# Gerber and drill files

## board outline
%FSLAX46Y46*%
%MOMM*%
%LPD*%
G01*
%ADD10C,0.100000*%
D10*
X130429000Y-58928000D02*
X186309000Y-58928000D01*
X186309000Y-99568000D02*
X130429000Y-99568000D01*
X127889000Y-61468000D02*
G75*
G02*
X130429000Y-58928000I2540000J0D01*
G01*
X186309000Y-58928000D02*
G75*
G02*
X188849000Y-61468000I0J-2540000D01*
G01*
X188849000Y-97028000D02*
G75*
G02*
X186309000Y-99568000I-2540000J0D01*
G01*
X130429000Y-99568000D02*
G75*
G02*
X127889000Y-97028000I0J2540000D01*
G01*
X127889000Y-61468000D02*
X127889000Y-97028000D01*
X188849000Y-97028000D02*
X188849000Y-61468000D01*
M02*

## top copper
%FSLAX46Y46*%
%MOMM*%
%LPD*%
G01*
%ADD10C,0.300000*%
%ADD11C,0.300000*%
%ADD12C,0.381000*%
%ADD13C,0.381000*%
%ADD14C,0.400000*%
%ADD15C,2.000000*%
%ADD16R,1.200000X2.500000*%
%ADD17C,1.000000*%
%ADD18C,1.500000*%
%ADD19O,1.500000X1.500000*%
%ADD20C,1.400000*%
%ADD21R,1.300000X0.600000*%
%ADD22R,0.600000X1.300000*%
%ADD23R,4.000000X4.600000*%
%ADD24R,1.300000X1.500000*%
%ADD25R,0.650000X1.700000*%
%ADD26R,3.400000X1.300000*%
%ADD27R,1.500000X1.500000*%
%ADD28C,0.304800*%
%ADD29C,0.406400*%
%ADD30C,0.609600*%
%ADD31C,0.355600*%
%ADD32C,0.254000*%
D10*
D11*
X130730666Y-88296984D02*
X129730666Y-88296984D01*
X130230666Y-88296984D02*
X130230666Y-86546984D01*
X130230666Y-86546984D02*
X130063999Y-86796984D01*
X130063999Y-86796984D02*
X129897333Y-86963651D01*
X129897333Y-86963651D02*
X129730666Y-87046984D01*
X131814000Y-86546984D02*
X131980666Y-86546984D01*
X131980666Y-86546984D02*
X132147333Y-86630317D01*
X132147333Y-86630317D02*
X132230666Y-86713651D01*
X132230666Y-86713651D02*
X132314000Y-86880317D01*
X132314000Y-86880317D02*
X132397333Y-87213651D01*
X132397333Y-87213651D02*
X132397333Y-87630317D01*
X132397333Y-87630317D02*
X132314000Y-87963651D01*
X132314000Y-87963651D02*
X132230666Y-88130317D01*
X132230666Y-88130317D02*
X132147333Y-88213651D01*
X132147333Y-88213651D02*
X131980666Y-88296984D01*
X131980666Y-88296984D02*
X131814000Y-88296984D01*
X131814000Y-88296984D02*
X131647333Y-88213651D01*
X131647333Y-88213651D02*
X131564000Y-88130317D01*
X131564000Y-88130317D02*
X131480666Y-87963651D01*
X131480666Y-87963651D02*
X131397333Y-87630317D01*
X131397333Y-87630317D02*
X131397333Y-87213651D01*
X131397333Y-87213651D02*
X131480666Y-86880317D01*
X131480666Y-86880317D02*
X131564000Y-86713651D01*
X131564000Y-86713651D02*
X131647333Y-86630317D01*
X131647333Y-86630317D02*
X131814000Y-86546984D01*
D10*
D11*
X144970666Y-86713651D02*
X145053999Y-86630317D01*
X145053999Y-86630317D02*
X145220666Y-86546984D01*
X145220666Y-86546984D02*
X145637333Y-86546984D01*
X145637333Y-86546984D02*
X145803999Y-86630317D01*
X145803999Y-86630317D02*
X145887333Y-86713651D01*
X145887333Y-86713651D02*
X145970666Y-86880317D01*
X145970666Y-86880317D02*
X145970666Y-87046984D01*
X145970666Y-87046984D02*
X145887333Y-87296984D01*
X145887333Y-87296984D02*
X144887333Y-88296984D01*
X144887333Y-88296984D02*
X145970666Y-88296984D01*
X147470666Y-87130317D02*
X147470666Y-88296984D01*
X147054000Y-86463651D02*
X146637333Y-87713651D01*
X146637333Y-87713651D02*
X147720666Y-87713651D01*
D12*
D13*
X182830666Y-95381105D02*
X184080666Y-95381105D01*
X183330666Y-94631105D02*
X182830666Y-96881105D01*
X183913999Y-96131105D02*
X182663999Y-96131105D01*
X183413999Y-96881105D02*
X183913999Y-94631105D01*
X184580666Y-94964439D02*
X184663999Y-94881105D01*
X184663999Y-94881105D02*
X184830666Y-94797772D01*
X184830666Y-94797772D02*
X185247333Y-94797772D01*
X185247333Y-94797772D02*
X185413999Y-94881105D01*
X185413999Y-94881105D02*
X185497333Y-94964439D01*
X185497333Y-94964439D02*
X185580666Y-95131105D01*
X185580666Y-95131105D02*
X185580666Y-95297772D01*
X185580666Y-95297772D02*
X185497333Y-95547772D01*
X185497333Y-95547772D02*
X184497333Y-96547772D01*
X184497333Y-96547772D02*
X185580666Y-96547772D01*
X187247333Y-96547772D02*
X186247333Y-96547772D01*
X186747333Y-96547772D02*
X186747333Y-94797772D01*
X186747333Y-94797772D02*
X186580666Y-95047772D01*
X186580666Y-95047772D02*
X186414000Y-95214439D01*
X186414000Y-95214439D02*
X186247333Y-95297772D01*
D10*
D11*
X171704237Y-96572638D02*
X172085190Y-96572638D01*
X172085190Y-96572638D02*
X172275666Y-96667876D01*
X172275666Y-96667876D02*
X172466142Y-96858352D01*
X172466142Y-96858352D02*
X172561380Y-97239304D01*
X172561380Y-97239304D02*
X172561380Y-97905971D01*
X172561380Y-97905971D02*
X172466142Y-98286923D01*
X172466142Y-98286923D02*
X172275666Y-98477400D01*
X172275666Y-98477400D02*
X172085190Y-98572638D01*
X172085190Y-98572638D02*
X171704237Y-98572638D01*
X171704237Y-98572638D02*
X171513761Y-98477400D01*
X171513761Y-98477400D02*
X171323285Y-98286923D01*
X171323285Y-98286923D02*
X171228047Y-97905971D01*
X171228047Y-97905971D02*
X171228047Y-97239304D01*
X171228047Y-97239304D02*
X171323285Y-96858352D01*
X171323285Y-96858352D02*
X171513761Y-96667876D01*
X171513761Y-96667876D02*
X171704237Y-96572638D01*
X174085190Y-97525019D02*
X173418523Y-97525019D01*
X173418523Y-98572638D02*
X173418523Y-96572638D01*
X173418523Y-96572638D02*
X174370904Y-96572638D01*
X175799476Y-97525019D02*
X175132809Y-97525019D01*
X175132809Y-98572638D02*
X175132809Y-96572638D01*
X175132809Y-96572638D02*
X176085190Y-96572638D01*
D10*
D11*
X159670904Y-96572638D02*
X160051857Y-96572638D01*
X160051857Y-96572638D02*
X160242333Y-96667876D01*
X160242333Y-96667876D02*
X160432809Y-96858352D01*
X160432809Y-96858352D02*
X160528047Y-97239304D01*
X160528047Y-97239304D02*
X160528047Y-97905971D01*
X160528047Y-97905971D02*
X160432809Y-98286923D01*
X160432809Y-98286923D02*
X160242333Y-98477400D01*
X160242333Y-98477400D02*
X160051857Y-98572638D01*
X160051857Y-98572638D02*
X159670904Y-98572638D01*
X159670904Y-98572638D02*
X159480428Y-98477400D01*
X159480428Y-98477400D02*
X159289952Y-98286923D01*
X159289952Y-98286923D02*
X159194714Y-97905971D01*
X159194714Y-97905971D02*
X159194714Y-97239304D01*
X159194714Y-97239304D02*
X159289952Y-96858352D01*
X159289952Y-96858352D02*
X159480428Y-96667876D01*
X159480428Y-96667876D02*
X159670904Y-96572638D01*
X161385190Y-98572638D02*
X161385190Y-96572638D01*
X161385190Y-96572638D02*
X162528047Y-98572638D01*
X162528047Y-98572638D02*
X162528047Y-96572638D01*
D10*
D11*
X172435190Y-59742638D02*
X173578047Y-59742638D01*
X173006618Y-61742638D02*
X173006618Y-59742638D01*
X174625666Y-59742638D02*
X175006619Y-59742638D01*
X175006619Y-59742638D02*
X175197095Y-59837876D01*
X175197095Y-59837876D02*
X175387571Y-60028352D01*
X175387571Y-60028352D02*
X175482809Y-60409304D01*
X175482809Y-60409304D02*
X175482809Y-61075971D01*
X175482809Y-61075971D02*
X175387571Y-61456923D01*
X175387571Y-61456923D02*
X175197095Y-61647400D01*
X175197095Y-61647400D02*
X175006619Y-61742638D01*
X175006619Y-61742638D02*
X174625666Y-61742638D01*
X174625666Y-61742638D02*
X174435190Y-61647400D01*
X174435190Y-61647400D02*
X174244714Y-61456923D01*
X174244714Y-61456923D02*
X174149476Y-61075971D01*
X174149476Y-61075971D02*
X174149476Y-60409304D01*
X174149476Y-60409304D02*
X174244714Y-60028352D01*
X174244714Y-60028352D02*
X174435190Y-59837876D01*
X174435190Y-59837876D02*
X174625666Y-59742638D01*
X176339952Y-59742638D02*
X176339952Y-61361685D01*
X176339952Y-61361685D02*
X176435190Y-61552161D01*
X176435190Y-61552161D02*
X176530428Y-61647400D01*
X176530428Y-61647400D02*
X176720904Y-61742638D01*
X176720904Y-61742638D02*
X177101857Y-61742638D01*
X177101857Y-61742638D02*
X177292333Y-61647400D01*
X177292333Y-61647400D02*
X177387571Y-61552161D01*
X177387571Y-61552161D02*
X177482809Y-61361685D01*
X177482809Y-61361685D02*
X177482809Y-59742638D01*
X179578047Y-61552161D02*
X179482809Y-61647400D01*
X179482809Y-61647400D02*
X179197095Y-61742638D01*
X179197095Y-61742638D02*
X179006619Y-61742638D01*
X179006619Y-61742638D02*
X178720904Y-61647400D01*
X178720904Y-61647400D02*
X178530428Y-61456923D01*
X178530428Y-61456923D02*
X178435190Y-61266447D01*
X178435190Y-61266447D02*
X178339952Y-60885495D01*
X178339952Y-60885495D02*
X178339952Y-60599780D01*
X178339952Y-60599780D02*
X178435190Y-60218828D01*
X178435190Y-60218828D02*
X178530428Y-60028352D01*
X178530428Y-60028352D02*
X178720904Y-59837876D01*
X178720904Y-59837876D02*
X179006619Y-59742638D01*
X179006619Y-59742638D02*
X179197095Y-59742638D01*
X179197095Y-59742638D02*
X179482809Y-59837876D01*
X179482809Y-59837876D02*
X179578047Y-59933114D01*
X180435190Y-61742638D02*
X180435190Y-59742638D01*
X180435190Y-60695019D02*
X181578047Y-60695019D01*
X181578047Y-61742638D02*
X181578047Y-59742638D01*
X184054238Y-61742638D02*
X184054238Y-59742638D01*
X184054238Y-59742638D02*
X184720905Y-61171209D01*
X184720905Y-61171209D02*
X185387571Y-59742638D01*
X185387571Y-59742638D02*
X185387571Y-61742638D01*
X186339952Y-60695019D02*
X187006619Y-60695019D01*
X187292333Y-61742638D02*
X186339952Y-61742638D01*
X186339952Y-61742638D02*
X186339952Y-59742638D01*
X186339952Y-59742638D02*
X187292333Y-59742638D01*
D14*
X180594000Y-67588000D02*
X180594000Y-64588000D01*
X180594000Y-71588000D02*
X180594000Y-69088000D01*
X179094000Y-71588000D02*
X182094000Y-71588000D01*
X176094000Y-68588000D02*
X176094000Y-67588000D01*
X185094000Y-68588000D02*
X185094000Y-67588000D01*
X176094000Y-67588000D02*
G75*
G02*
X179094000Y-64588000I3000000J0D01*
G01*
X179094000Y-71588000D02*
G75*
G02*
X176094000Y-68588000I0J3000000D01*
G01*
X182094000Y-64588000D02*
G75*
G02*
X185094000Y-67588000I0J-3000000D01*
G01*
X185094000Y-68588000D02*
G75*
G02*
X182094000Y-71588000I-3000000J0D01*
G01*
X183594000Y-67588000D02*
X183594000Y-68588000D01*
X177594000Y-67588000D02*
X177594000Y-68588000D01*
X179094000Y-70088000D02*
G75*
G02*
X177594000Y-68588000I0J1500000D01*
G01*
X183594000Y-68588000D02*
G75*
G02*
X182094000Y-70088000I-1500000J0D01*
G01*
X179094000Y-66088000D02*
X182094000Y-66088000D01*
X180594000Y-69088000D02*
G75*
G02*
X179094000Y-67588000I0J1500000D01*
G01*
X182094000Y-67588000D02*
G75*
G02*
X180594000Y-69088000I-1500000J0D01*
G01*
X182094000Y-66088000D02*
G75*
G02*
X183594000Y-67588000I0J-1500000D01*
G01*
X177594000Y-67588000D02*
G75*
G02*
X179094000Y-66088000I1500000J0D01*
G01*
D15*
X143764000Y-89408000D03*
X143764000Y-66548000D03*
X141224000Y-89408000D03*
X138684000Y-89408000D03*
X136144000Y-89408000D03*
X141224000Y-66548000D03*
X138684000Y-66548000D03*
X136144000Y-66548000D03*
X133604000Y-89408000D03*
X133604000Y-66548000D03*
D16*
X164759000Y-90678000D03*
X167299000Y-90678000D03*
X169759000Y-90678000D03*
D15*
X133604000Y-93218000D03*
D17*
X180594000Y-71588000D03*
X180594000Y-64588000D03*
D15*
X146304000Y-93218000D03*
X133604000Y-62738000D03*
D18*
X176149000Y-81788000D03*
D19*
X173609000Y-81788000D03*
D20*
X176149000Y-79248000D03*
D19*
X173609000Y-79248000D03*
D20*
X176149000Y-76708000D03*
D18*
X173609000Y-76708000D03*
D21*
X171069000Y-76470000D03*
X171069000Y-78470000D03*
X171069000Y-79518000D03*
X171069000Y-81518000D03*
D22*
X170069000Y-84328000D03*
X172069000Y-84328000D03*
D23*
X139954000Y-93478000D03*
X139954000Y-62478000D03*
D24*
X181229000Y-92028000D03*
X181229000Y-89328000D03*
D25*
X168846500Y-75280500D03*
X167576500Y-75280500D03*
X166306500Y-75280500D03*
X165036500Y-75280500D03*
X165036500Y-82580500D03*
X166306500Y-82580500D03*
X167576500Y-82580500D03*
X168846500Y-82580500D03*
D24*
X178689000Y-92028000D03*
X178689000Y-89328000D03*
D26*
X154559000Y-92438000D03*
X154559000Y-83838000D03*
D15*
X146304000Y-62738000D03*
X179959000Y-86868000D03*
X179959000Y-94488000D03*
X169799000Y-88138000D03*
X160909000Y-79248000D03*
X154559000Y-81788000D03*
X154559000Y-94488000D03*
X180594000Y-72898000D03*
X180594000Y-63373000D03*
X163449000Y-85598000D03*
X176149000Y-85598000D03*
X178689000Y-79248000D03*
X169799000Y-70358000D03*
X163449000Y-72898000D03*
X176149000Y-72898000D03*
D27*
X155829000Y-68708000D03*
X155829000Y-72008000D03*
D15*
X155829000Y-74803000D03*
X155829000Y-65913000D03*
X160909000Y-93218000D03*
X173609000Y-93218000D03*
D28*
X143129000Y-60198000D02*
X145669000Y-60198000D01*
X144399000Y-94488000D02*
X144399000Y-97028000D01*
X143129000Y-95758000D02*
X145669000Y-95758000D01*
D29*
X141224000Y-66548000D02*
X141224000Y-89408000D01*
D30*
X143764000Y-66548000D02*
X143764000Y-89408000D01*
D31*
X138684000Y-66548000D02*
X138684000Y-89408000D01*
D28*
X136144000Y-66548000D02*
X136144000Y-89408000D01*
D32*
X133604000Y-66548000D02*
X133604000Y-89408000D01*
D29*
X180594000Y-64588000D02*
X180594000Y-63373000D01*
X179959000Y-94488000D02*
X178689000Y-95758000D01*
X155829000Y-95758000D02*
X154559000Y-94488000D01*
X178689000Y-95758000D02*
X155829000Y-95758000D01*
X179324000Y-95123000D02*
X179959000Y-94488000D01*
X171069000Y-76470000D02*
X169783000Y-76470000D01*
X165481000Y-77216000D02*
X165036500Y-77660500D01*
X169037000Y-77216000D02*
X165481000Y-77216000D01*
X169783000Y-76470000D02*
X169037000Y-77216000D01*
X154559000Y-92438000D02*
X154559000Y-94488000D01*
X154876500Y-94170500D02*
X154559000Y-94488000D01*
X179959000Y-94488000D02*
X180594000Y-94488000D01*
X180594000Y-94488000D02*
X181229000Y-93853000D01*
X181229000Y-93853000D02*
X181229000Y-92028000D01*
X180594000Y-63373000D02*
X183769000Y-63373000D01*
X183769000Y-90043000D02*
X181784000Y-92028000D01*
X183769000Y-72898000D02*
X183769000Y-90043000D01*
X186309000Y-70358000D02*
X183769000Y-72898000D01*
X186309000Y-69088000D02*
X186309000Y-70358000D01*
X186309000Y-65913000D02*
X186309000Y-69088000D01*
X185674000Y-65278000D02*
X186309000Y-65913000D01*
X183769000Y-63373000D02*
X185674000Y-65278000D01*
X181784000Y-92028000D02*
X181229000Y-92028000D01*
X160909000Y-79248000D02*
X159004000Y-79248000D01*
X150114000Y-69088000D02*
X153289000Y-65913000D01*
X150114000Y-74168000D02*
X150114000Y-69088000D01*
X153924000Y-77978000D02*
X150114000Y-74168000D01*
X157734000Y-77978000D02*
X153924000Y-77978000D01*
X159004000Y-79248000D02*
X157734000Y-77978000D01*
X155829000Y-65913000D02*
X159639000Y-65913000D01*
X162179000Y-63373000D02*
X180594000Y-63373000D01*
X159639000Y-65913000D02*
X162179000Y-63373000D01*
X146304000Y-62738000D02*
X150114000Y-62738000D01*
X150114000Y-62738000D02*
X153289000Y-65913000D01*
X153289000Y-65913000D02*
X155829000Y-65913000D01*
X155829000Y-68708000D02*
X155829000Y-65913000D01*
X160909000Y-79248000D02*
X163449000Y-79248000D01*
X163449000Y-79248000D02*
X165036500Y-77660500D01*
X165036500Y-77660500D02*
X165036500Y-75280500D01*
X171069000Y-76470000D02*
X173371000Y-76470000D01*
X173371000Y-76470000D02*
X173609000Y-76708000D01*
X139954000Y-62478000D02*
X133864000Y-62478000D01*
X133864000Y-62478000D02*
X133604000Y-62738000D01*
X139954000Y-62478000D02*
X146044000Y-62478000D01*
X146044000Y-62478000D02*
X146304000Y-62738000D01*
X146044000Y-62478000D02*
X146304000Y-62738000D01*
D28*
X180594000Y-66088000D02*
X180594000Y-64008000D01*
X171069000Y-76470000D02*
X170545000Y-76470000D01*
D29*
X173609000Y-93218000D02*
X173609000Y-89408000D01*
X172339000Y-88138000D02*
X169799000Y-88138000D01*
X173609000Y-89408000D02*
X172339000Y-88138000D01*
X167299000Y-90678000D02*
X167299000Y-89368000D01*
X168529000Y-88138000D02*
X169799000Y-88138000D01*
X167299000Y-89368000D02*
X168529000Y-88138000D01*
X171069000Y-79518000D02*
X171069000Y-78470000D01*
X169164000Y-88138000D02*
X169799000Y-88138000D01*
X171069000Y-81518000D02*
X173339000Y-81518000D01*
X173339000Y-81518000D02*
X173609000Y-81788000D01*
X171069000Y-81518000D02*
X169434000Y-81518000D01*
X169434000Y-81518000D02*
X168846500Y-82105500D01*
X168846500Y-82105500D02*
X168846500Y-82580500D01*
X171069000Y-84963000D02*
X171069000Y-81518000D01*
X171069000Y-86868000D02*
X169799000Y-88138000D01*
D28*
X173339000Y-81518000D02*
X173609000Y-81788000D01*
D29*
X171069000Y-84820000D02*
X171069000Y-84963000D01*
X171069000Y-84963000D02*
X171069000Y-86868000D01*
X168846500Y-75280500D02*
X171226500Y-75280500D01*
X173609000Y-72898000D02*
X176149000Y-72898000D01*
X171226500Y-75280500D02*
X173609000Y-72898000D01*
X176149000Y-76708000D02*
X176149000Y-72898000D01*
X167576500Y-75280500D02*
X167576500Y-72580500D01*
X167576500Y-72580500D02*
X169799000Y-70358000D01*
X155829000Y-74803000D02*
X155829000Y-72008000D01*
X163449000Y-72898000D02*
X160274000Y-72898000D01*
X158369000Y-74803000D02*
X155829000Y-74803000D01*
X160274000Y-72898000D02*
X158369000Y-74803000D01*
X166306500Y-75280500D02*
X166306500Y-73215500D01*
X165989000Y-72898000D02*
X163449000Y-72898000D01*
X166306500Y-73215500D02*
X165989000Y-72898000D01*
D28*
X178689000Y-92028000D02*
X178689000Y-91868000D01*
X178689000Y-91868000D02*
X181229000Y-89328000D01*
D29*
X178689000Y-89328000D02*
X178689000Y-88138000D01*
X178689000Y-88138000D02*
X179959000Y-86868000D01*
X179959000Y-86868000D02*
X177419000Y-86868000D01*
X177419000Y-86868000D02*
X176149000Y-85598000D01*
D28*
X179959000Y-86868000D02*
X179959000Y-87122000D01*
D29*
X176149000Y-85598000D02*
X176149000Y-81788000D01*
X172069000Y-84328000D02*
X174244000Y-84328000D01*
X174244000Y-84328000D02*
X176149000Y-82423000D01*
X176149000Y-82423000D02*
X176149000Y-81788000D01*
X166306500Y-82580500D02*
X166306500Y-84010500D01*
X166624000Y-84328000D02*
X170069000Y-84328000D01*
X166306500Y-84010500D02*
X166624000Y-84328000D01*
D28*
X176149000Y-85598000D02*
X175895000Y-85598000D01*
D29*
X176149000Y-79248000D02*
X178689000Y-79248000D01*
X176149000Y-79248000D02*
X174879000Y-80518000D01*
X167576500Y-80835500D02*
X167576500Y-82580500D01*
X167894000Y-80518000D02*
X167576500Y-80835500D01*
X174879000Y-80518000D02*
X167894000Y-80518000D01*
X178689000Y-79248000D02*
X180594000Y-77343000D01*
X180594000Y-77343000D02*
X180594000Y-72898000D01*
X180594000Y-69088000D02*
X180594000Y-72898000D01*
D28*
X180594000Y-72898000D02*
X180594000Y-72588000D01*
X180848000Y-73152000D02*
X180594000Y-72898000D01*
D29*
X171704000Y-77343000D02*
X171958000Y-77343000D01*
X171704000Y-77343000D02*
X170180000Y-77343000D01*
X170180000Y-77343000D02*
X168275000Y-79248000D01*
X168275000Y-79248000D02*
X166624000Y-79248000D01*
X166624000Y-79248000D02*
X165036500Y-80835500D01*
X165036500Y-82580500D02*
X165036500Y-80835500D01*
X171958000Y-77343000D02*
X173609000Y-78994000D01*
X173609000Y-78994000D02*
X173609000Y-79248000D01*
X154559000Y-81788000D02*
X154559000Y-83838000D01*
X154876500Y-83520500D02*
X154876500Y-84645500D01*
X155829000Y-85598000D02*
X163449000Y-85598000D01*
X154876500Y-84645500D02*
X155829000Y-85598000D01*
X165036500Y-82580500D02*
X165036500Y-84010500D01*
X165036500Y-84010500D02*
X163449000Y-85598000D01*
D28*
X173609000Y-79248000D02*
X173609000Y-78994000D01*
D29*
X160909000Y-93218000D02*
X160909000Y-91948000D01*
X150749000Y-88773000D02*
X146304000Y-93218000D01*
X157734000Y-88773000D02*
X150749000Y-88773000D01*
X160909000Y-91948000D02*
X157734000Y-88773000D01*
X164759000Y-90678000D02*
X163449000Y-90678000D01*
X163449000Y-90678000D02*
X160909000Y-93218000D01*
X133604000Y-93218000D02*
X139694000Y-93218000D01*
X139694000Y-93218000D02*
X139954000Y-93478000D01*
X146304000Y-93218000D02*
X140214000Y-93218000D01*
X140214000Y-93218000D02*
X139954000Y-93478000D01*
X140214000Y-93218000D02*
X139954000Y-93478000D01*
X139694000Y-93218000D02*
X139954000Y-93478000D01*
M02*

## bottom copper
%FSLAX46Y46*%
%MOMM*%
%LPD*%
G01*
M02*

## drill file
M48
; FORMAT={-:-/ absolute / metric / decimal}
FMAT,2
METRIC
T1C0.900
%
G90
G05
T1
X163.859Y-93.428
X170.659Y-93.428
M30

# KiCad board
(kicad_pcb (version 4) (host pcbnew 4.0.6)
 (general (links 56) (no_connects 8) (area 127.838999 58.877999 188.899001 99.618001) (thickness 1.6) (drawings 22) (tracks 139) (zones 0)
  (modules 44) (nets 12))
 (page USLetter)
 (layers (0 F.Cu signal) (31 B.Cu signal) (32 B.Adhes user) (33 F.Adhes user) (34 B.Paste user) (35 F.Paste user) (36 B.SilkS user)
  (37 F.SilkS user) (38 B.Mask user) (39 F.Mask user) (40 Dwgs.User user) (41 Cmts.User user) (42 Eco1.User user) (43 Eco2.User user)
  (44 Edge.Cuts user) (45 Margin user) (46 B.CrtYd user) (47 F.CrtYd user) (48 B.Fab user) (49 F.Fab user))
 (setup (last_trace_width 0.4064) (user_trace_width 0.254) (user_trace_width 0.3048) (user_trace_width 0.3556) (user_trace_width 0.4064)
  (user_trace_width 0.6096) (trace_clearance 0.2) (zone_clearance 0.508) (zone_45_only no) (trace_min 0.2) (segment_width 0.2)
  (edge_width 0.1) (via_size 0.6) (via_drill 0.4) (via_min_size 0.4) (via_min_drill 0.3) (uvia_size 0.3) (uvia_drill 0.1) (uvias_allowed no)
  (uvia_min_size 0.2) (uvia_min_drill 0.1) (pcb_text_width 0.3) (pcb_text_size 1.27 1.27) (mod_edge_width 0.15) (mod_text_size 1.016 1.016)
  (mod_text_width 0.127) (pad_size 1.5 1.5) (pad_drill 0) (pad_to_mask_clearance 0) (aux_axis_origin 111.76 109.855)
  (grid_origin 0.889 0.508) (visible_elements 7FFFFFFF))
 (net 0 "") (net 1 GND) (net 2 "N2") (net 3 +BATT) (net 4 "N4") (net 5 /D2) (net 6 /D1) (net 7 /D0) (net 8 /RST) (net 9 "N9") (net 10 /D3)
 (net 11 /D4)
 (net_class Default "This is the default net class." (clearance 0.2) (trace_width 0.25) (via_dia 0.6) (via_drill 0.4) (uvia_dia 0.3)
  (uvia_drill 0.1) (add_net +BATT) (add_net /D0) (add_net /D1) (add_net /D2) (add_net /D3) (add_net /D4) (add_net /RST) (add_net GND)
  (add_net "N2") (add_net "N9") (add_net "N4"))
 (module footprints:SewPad (layer F.Cu) (at 143.764 89.408)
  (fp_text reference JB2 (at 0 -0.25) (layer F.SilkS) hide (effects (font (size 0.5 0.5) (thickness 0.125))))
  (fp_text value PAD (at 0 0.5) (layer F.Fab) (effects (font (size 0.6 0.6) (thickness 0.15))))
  (pad 1 smd circle (at 0 0) (size 2 2) (layers F.Cu F.Mask) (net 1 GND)))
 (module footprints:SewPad (layer F.Cu) (at 143.764 66.548)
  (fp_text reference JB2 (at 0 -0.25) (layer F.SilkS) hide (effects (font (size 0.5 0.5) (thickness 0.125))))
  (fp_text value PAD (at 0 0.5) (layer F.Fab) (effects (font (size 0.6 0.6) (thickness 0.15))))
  (pad 1 smd circle (at 0 0) (size 2 2) (layers F.Cu F.Mask) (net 1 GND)))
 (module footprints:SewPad (layer F.Cu) (at 141.224 89.408)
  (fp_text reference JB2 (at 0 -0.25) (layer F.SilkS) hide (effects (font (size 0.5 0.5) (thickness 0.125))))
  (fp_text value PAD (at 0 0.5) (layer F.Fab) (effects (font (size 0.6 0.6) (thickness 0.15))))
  (pad 1 smd circle (at 0 0) (size 2 2) (layers F.Cu F.Mask) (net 1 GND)))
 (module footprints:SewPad (layer F.Cu) (at 138.684 89.408)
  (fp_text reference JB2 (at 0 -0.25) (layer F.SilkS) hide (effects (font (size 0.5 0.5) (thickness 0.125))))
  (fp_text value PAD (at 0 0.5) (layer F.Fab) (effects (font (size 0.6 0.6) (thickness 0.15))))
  (pad 1 smd circle (at 0 0) (size 2 2) (layers F.Cu F.Mask) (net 1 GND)))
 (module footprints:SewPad (layer F.Cu) (at 136.144 89.408)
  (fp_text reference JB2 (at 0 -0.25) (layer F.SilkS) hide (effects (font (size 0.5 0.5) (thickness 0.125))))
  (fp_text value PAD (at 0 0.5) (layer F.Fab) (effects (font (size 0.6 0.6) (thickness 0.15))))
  (pad 1 smd circle (at 0 0) (size 2 2) (layers F.Cu F.Mask) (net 1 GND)))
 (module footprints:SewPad (layer F.Cu) (at 141.224 66.548)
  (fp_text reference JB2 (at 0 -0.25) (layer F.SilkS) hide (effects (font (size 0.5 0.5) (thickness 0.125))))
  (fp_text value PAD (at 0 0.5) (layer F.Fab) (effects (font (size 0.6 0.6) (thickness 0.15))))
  (pad 1 smd circle (at 0 0) (size 2 2) (layers F.Cu F.Mask) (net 1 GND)))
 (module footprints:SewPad (layer F.Cu) (at 138.684 66.548)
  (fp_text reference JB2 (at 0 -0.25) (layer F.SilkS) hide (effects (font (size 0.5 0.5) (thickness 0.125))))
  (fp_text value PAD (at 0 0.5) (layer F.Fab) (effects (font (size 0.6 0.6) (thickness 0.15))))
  (pad 1 smd circle (at 0 0) (size 2 2) (layers F.Cu F.Mask) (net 1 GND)))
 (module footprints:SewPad (layer F.Cu) (at 136.144 66.548)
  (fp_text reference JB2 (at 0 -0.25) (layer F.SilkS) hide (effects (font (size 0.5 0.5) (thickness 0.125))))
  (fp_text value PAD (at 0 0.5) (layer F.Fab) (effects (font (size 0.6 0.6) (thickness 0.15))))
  (pad 1 smd circle (at 0 0) (size 2 2) (layers F.Cu F.Mask) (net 1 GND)))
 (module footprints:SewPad (layer F.Cu) (at 133.604 89.408)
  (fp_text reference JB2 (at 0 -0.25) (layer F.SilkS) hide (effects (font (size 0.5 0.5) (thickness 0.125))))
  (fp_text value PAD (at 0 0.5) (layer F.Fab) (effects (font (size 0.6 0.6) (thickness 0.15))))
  (pad 1 smd circle (at 0 0) (size 2 2) (layers F.Cu F.Mask) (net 1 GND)))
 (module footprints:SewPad (layer F.Cu) (at 133.604 66.548)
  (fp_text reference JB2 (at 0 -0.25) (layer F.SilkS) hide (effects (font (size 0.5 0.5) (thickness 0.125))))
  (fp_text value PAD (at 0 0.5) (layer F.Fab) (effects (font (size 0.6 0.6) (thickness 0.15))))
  (pad 1 smd circle (at 0 0) (size 2 2) (layers F.Cu F.Mask) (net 1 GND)))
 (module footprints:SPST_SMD (layer F.Cu) (at 167.259 90.678)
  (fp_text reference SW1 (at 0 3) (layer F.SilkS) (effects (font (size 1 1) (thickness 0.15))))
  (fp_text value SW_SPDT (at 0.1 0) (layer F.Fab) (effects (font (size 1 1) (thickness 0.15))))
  (pad "" np_thru_hole circle (at 3.4 2.75) (size 0.9 0.9) (drill 0.9) (layers *.Cu *.Mask))
  (pad 1 smd rect (at -2.5 0) (size 1.2 2.5) (layers F.Cu F.Paste F.Mask) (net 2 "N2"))
  (pad 2 smd rect (at 0.04 0) (size 1.2 2.5) (layers F.Cu F.Paste F.Mask) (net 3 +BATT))
  (pad 3 smd rect (at 2.5 0) (size 1.2 2.5) (layers F.Cu F.Paste F.Mask) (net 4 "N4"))
  (pad "" np_thru_hole circle (at -3.4 2.75) (size 0.9 0.9) (drill 0.9) (layers *.Cu *.Mask)))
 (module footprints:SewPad (layer F.Cu) (at 133.604 93.218)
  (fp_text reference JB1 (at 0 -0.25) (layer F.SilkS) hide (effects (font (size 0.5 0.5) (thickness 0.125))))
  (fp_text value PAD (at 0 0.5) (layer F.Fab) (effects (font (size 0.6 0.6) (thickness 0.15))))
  (pad 1 smd circle (at 0 0) (size 2 2) (layers F.Cu F.Mask) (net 2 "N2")))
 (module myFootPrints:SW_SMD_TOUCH (layer F.Cu) (at 180.594 69.088)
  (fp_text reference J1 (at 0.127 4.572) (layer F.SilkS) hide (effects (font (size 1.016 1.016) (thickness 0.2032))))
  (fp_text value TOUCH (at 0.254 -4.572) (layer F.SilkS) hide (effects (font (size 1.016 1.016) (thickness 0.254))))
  (fp_line (start 0 -1.5) (end 0 -4.5) (layer F.Cu) (width 0.4)) (fp_line (start 0 2.5) (end 0 0) (layer F.Cu) (width 0.4))
  (fp_line (start -1.5 2.5) (end 1.5 2.5) (layer F.Cu) (width 0.4))
  (fp_line (start -4.5 -0.5) (end -4.5 -1.5) (layer F.Cu) (width 0.4))
  (fp_line (start 4.5 -0.5) (end 4.5 -1.5) (layer F.Cu) (width 0.4))
  (fp_arc (start -1.5 -1.5) (end -4.5 -1.5) (angle 90) (layer F.Cu) (width 0.4))
  (fp_arc (start -1.5 -0.5) (end -1.5 2.5) (angle 90) (layer F.Cu) (width 0.4))
  (fp_arc (start 1.5 -1.5) (end 1.5 -4.5) (angle 90) (layer F.Cu) (width 0.4))
  (fp_arc (start 1.5 -0.5) (end 4.5 -0.5) (angle 90) (layer F.Cu) (width 0.4))
  (fp_line (start 3 -1.5) (end 3 -0.5) (layer F.Cu) (width 0.4))
  (fp_line (start -3 -1.5) (end -3 -0.5) (layer F.Cu) (width 0.4))
  (fp_arc (start -1.5 -0.5) (end -1.5 1) (angle 90) (layer F.Cu) (width 0.4))
  (fp_arc (start 1.5 -0.5) (end 3 -0.5) (angle 90) (layer F.Cu) (width 0.4))
  (fp_line (start -1.5 -3) (end 1.5 -3) (layer F.Cu) (width 0.4))
  (fp_arc (start 0 -1.5) (end 0 0) (angle 90) (layer F.Cu) (width 0.4))
  (fp_arc (start 0 -1.5) (end 1.5 -1.5) (angle 90) (layer F.Cu) (width 0.4))
  (fp_arc (start 1.5 -1.5) (end 1.5 -3) (angle 90) (layer F.Cu) (width 0.4))
  (fp_arc (start -1.5 -1.5) (end -3 -1.5) (angle 90) (layer F.Cu) (width 0.4))
  (pad 2 smd circle (at 0 2.5) (size 1 1) (layers F.Cu) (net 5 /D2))
  (pad 1 smd circle (at 0 -4.5) (size 1 1) (layers F.Cu) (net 1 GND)))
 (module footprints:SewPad (layer F.Cu) (at 146.304 93.218)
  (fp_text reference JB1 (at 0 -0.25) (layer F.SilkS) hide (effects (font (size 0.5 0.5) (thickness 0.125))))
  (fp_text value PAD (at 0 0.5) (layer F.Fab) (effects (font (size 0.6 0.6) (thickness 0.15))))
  (pad 1 smd circle (at 0 0) (size 2 2) (layers F.Cu F.Mask) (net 2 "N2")))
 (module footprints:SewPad (layer F.Cu) (at 133.604 62.738)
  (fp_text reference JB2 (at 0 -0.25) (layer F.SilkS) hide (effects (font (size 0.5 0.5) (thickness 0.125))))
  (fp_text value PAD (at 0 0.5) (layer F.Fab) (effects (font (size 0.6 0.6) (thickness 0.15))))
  (pad 1 smd circle (at 0 0) (size 2 2) (layers F.Cu F.Mask) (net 1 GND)))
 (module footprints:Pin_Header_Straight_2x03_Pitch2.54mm (layer F.Cu) (at 176.149 81.788 180)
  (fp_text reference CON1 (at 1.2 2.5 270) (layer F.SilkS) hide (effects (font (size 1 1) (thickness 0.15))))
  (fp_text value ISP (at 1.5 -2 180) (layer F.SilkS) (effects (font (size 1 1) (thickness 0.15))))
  (pad 1 smd circle (at 0 0 180) (size 1.5 1.5) (layers F.Cu) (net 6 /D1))
  (pad 2 smd oval (at 2.54 0 180) (size 1.5 1.5) (layers F.Cu) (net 3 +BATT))
  (pad 3 smd circle (at 0 2.54 180) (size 1.4 1.4) (layers F.Cu) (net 5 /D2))
  (pad 4 smd oval (at 2.54 2.54 180) (size 1.5 1.5) (layers F.Cu) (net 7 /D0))
  (pad 5 smd circle (at 0 5.08 180) (size 1.4 1.4) (layers F.Cu) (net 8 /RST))
  (pad 6 smd circle (at 2.54 5.08 180) (size 1.5 1.5) (layers F.Cu) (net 1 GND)))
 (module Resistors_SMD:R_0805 (layer F.Cu) (at 171.069 77.47 270)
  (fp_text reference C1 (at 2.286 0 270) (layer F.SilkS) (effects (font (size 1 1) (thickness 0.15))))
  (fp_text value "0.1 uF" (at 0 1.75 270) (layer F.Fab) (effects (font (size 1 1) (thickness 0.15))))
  (pad 1 smd rect (at -1 0 270) (size 0.6 1.3) (layers F.Cu F.Paste F.Mask) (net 1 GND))
  (pad 2 smd rect (at 1 0 270) (size 0.6 1.3) (layers F.Cu F.Paste F.Mask) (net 3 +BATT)))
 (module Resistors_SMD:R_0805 (layer F.Cu) (at 171.069 80.518 270)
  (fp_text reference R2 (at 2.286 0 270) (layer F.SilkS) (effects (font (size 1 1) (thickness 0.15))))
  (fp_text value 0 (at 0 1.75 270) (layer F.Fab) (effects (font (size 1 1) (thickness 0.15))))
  (pad 1 smd rect (at -1 0 270) (size 0.6 1.3) (layers F.Cu F.Paste F.Mask) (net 3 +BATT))
  (pad 2 smd rect (at 1 0 270) (size 0.6 1.3) (layers F.Cu F.Paste F.Mask) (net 3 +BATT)))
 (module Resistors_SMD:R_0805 (layer F.Cu) (at 171.069 84.328)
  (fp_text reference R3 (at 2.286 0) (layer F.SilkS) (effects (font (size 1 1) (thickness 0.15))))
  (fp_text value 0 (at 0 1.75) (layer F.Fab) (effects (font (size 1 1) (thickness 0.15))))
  (pad 1 smd rect (at -1 0) (size 0.6 1.3) (layers F.Cu F.Paste F.Mask) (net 6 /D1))
  (pad 2 smd rect (at 1 0) (size 0.6 1.3) (layers F.Cu F.Paste F.Mask) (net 6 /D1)))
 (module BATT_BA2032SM (layer F.Cu) (at 139.954 77.978 90)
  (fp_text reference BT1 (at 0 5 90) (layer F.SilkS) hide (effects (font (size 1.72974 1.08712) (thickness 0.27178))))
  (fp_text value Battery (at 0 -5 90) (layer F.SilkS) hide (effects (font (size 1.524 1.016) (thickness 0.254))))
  (pad 1 smd rect (at -15.5 0 90) (size 4.6 4) (layers F.Cu F.Paste F.Mask) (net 2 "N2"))
  (pad 2 smd rect (at 15.5 0 90) (size 4.6 4) (layers F.Cu F.Paste F.Mask) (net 1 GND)))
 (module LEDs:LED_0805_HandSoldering (layer F.Cu) (at 181.229 90.678 90)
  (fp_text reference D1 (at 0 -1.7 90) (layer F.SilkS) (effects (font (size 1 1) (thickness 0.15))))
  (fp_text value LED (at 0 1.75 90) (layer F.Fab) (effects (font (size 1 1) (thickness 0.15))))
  (pad 1 smd rect (at -1.35 0 90) (size 1.5 1.3) (layers F.Cu F.Paste F.Mask) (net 1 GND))
  (pad 2 smd rect (at 1.35 0 90) (size 1.5 1.3) (layers F.Cu F.Paste F.Mask) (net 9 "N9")))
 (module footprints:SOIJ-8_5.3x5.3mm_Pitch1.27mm (layer F.Cu) (at 166.9415 78.9305 270)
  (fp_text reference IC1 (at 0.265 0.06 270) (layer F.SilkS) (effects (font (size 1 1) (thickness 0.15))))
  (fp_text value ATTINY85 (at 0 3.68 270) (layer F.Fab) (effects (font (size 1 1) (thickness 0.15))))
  (pad 1 smd rect (at -3.65 -1.905 270) (size 1.7 0.65) (layers F.Cu F.Paste F.Mask) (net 8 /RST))
  (pad 2 smd rect (at -3.65 -0.635 270) (size 1.7 0.65) (layers F.Cu F.Paste F.Mask) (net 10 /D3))
  (pad 3 smd rect (at -3.65 0.635 270) (size 1.7 0.65) (layers F.Cu F.Paste F.Mask) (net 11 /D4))
  (pad 4 smd rect (at -3.65 1.905 270) (size 1.7 0.65) (layers F.Cu F.Paste F.Mask) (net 1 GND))
  (pad 5 smd rect (at 3.65 1.905 270) (size 1.7 0.65) (layers F.Cu F.Paste F.Mask) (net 7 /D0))
  (pad 6 smd rect (at 3.65 0.635 270) (size 1.7 0.65) (layers F.Cu F.Paste F.Mask) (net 6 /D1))
  (pad 7 smd rect (at 3.65 -0.635 270) (size 1.7 0.65) (layers F.Cu F.Paste F.Mask) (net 5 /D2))
  (pad 8 smd rect (at 3.65 -1.905 270) (size 1.7 0.65) (layers F.Cu F.Paste F.Mask) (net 3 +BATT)))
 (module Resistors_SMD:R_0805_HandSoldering (layer F.Cu) (at 178.689 90.678 90)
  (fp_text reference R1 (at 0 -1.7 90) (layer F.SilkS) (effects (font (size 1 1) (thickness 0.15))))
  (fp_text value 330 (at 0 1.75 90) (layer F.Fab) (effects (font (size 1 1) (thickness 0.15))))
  (pad 1 smd rect (at -1.35 0 90) (size 1.5 1.3) (layers F.Cu F.Paste F.Mask) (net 9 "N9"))
  (pad 2 smd rect (at 1.35 0 90) (size 1.5 1.3) (layers F.Cu F.Paste F.Mask) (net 6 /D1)))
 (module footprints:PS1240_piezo (layer F.Cu) (at 154.559 88.138 90)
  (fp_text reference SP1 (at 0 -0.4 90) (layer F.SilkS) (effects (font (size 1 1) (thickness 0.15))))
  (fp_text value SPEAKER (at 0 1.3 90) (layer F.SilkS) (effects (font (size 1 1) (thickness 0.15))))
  (pad 1 smd rect (at -4.3 0 90) (size 1.3 3.4) (layers F.Cu F.Paste F.Mask) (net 1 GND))
  (pad 2 smd rect (at 4.3 0 90) (size 1.3 3.4) (layers F.Cu F.Paste F.Mask) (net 7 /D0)))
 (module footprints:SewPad (layer F.Cu) (at 146.304 62.738)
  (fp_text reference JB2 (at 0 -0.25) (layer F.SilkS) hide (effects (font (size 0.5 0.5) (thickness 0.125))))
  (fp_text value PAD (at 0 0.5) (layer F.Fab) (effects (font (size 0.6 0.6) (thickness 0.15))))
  (pad 1 smd circle (at 0 0) (size 2 2) (layers F.Cu F.Mask) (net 1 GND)))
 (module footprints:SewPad (layer F.Cu) (at 179.959 86.868 90)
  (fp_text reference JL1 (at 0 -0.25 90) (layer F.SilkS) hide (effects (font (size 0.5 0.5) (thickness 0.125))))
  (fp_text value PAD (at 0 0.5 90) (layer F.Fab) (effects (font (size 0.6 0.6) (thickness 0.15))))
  (pad 1 smd circle (at 0 0 90) (size 2 2) (layers F.Cu F.Mask) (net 6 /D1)))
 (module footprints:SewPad (layer F.Cu) (at 179.959 94.488 90)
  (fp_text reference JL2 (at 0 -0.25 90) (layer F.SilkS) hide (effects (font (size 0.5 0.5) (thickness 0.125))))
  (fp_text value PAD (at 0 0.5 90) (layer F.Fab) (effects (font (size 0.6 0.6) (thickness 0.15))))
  (pad 1 smd circle (at 0 0 90) (size 2 2) (layers F.Cu F.Mask) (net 1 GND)))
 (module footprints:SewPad (layer F.Cu) (at 169.799 88.138)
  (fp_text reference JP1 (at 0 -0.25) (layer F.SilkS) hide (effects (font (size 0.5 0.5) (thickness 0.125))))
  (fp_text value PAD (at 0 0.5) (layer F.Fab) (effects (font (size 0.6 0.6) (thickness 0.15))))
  (pad 1 smd circle (at 0 0) (size 2 2) (layers F.Cu F.Mask) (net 3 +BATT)))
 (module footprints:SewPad (layer F.Cu) (at 160.909 79.248)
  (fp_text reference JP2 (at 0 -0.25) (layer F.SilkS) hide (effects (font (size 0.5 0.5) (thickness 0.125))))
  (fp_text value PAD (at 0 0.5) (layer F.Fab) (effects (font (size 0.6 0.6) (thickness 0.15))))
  (pad 1 smd circle (at 0 0) (size 2 2) (layers F.Cu F.Mask) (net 1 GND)))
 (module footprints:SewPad (layer F.Cu) (at 154.559 81.788 180)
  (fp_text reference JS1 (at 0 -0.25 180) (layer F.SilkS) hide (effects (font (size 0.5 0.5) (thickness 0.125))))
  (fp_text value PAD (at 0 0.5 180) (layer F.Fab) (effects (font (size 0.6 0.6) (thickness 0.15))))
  (pad 1 smd circle (at 0 0 180) (size 2 2) (layers F.Cu F.Mask) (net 7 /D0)))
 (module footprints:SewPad (layer F.Cu) (at 154.559 94.488 180)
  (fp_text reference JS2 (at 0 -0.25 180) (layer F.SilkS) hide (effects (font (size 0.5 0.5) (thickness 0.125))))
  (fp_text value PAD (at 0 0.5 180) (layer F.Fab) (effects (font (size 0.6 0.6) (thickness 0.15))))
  (pad 1 smd circle (at 0 0 180) (size 2 2) (layers F.Cu F.Mask) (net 1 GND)))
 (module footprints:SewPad (layer F.Cu) (at 180.594 72.898 90)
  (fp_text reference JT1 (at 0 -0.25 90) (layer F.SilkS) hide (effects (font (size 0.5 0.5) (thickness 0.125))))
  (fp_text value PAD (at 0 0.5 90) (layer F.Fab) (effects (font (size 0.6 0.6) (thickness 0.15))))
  (pad 1 smd circle (at 0 0 90) (size 2 2) (layers F.Cu F.Mask) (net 5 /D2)))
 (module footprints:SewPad (layer F.Cu) (at 180.594 63.373 90)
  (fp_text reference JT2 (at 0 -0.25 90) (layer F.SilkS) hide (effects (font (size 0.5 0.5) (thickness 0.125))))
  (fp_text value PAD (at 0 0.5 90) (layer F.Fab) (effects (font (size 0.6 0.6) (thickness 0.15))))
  (pad 1 smd circle (at 0 0 90) (size 2 2) (layers F.Cu F.Mask) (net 1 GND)))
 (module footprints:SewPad (layer F.Cu) (at 163.449 85.598)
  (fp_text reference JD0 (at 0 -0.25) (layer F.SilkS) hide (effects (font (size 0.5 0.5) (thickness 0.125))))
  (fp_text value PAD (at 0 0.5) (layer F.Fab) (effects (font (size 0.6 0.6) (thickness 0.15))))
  (pad 1 smd circle (at 0 0) (size 2 2) (layers F.Cu F.Mask) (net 7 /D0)))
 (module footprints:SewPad (layer F.Cu) (at 176.149 85.598)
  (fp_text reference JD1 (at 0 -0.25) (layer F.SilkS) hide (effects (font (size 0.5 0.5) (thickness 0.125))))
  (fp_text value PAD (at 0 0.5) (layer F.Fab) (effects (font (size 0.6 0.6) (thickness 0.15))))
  (pad 1 smd circle (at 0 0) (size 2 2) (layers F.Cu F.Mask) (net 6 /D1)))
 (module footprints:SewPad (layer F.Cu) (at 178.689 79.248)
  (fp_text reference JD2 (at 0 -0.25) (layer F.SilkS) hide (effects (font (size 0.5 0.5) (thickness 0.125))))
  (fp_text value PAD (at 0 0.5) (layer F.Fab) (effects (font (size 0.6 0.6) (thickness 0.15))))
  (pad 1 smd circle (at 0 0) (size 2 2) (layers F.Cu F.Mask) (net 5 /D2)))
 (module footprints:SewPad (layer F.Cu) (at 169.799 70.358)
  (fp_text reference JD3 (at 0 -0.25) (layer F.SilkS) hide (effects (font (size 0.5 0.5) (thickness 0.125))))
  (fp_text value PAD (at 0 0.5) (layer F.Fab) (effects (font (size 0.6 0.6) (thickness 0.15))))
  (pad 1 smd circle (at 0 0) (size 2 2) (layers F.Cu F.Mask) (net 10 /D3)))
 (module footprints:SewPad (layer F.Cu) (at 163.449 72.898)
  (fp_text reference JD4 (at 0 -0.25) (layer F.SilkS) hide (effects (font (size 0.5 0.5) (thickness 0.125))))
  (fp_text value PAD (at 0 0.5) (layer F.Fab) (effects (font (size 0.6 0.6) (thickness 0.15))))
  (pad 1 smd circle (at 0 0) (size 2 2) (layers F.Cu F.Mask) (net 11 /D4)))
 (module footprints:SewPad (layer F.Cu) (at 176.149 72.898)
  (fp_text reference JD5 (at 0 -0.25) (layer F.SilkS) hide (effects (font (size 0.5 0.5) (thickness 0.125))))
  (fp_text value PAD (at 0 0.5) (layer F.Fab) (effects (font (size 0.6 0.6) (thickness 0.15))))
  (pad 1 smd circle (at 0 0) (size 2 2) (layers F.Cu F.Mask) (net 8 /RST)))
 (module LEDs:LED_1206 (layer F.Cu) (at 155.829 70.358 90)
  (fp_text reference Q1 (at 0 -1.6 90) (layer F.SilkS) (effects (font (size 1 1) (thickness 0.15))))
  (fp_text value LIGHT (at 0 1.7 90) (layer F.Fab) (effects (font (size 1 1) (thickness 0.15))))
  (pad 2 smd rect (at 1.65 0 270) (size 1.5 1.5) (layers F.Cu F.Paste F.Mask) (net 1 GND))
  (pad 1 smd rect (at -1.65 0 270) (size 1.5 1.5) (layers F.Cu F.Paste F.Mask) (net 11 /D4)))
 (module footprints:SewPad (layer F.Cu) (at 155.829 74.803)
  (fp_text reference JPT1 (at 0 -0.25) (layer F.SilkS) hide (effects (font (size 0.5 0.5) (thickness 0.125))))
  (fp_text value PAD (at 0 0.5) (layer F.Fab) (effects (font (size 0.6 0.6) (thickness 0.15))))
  (pad 1 smd circle (at 0 0) (size 2 2) (layers F.Cu F.Mask) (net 11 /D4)))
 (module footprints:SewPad (layer F.Cu) (at 155.829 65.913)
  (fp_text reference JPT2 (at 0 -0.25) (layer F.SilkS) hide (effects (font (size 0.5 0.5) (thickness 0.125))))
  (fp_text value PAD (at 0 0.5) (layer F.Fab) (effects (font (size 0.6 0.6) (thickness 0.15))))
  (pad 1 smd circle (at 0 0) (size 2 2) (layers F.Cu F.Mask) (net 1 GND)))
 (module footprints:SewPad (layer F.Cu) (at 160.909 93.218)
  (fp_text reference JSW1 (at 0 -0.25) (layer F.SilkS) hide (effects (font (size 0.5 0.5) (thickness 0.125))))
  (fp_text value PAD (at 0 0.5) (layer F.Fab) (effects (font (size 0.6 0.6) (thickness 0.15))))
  (pad 1 smd circle (at 0 0) (size 2 2) (layers F.Cu F.Mask) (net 2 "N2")))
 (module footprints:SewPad (layer F.Cu) (at 173.609 93.218)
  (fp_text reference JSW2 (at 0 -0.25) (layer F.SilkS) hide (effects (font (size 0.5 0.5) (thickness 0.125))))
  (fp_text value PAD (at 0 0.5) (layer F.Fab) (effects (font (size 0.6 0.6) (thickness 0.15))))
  (pad 1 smd circle (at 0 0) (size 2 2) (layers F.Cu F.Mask) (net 3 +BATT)))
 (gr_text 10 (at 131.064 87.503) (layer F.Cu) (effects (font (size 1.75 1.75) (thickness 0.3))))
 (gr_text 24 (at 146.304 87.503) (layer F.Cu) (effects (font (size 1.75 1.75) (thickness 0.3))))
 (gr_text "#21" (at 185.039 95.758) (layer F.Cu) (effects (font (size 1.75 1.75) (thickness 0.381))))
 (gr_line (start 130.429 58.928) (end 186.309 58.928) (angle 90) (layer Edge.Cuts) (width 0.1))
 (gr_line (start 186.309 99.568) (end 130.429 99.568) (angle 90) (layer Edge.Cuts) (width 0.1))
 (gr_arc (start 130.429 61.468) (end 127.889 61.468) (angle 90) (layer Edge.Cuts) (width 0.1))
 (gr_arc (start 186.309 61.468) (end 186.309 58.928) (angle 90) (layer Edge.Cuts) (width 0.1))
 (gr_arc (start 186.309 97.028) (end 188.849 97.028) (angle 90) (layer Edge.Cuts) (width 0.1))
 (gr_arc (start 130.429 97.028) (end 130.429 99.568) (angle 90) (layer Edge.Cuts) (width 0.1))
 (gr_line (start 127.889 61.468) (end 127.889 97.028) (angle 90) (layer Edge.Cuts) (width 0.1))
 (gr_line (start 188.849 97.028) (end 188.849 61.468) (angle 90) (layer Edge.Cuts) (width 0.1))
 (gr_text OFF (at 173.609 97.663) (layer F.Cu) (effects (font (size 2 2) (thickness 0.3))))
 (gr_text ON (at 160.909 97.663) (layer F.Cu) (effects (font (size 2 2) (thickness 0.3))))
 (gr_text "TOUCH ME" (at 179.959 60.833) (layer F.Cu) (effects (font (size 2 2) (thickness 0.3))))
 (segment (start 143.129 60.198) (end 145.669 60.198) (width 0.3048) (layer F.Cu) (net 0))
 (segment (start 144.399 94.488) (end 144.399 97.028) (width 0.3048) (layer F.Cu) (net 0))
 (segment (start 143.129 95.758) (end 145.669 95.758) (width 0.3048) (layer F.Cu) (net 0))
 (segment (start 141.224 66.548) (end 141.224 89.408) (width 0.4064) (layer F.Cu) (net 1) (status C00000))
 (segment (start 143.764 66.548) (end 143.764 89.408) (width 0.6096) (layer F.Cu) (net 1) (status C00000))
 (segment (start 138.684 66.548) (end 138.684 89.408) (width 0.3556) (layer F.Cu) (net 1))
 (segment (start 136.144 66.548) (end 136.144 89.408) (width 0.3048) (layer F.Cu) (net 1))
 (segment (start 133.604 66.548) (end 133.604 89.408) (width 0.254) (layer F.Cu) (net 1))
 (segment (start 180.594 64.588) (end 180.594 63.373) (width 0.4064) (layer F.Cu) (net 1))
 (segment (start 179.959 94.488) (end 178.689 95.758) (width 0.4064) (layer F.Cu) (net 1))
 (segment (start 155.829 95.758) (end 154.559 94.488) (width 0.4064) (layer F.Cu) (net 1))
 (segment (start 178.689 95.758) (end 155.829 95.758) (width 0.4064) (layer F.Cu) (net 1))
 (segment (start 179.324 95.123) (end 179.959 94.488) (width 0.4064) (layer F.Cu) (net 1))
 (segment (start 171.069 76.47) (end 169.783 76.47) (width 0.4064) (layer F.Cu) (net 1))
 (segment (start 165.481 77.216) (end 165.0365 77.6605) (width 0.4064) (layer F.Cu) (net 1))
 (segment (start 169.037 77.216) (end 165.481 77.216) (width 0.4064) (layer F.Cu) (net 1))
 (segment (start 169.783 76.47) (end 169.037 77.216) (width 0.4064) (layer F.Cu) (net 1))
 (segment (start 154.559 92.438) (end 154.559 94.488) (width 0.4064) (layer F.Cu) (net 1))
 (segment (start 154.8765 94.1705) (end 154.559 94.488) (width 0.4064) (layer F.Cu) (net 1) (status 30))
 (segment (start 179.959 94.488) (end 180.594 94.488) (width 0.4064) (layer F.Cu) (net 1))
 (segment (start 180.594 94.488) (end 181.229 93.853) (width 0.4064) (layer F.Cu) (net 1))
 (segment (start 181.229 93.853) (end 181.229 92.028) (width 0.4064) (layer F.Cu) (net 1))
 (segment (start 180.594 63.373) (end 183.769 63.373) (width 0.4064) (layer F.Cu) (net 1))
 (segment (start 183.769 90.043) (end 181.784 92.028) (width 0.4064) (layer F.Cu) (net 1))
 (segment (start 183.769 72.898) (end 183.769 90.043) (width 0.4064) (layer F.Cu) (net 1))
 (segment (start 186.309 70.358) (end 183.769 72.898) (width 0.4064) (layer F.Cu) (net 1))
 (segment (start 186.309 69.088) (end 186.309 70.358) (width 0.4064) (layer F.Cu) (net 1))
 (segment (start 186.309 65.913) (end 186.309 69.088) (width 0.4064) (layer F.Cu) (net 1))
 (segment (start 185.674 65.278) (end 186.309 65.913) (width 0.4064) (layer F.Cu) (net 1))
 (segment (start 183.769 63.373) (end 185.674 65.278) (width 0.4064) (layer F.Cu) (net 1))
 (segment (start 181.784 92.028) (end 181.229 92.028) (width 0.4064) (layer F.Cu) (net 1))
 (segment (start 160.909 79.248) (end 159.004 79.248) (width 0.4064) (layer F.Cu) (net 1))
 (segment (start 150.114 69.088) (end 153.289 65.913) (width 0.4064) (layer F.Cu) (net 1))
 (segment (start 150.114 74.168) (end 150.114 69.088) (width 0.4064) (layer F.Cu) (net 1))
 (segment (start 153.924 77.978) (end 150.114 74.168) (width 0.4064) (layer F.Cu) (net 1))
 (segment (start 157.734 77.978) (end 153.924 77.978) (width 0.4064) (layer F.Cu) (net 1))
 (segment (start 159.004 79.248) (end 157.734 77.978) (width 0.4064) (layer F.Cu) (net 1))
 (segment (start 155.829 65.913) (end 159.639 65.913) (width 0.4064) (layer F.Cu) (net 1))
 (segment (start 162.179 63.373) (end 180.594 63.373) (width 0.4064) (layer F.Cu) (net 1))
 (segment (start 159.639 65.913) (end 162.179 63.373) (width 0.4064) (layer F.Cu) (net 1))
 (segment (start 146.304 62.738) (end 150.114 62.738) (width 0.4064) (layer F.Cu) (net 1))
 (segment (start 150.114 62.738) (end 153.289 65.913) (width 0.4064) (layer F.Cu) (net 1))
 (segment (start 153.289 65.913) (end 155.829 65.913) (width 0.4064) (layer F.Cu) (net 1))
 (segment (start 155.829 68.708) (end 155.829 65.913) (width 0.4064) (layer F.Cu) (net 1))
 (segment (start 160.909 79.248) (end 163.449 79.248) (width 0.4064) (layer F.Cu) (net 1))
 (segment (start 163.449 79.248) (end 165.0365 77.6605) (width 0.4064) (layer F.Cu) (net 1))
 (segment (start 165.0365 77.6605) (end 165.0365 75.2805) (width 0.4064) (layer F.Cu) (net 1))
 (segment (start 171.069 76.47) (end 173.371 76.47) (width 0.4064) (layer F.Cu) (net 1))
 (segment (start 173.371 76.47) (end 173.609 76.708) (width 0.4064) (layer F.Cu) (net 1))
 (segment (start 139.954 62.478) (end 133.864 62.478) (width 0.4064) (layer F.Cu) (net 1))
 (segment (start 133.864 62.478) (end 133.604 62.738) (width 0.4064) (layer F.Cu) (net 1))
 (segment (start 139.954 62.478) (end 146.044 62.478) (width 0.4064) (layer F.Cu) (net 1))
 (segment (start 146.044 62.478) (end 146.304 62.738) (width 0.4064) (layer F.Cu) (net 1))
 (segment (start 146.044 62.478) (end 146.304 62.738) (width 0.4064) (layer F.Cu) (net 1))
 (segment (start 180.594 66.088) (end 180.594 64.008) (width 0.3048) (layer F.Cu) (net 1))
 (segment (start 171.069 76.47) (end 170.545 76.47) (width 0.3048) (layer F.Cu) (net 1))
 (segment (start 173.609 93.218) (end 173.609 89.408) (width 0.4064) (layer F.Cu) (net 3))
 (segment (start 172.339 88.138) (end 169.799 88.138) (width 0.4064) (layer F.Cu) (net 3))
 (segment (start 173.609 89.408) (end 172.339 88.138) (width 0.4064) (layer F.Cu) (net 3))
 (segment (start 167.299 90.678) (end 167.299 89.368) (width 0.4064) (layer F.Cu) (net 3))
 (segment (start 168.529 88.138) (end 169.799 88.138) (width 0.4064) (layer F.Cu) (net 3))
 (segment (start 167.299 89.368) (end 168.529 88.138) (width 0.4064) (layer F.Cu) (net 3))
 (segment (start 171.069 79.518) (end 171.069 78.47) (width 0.4064) (layer F.Cu) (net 3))
 (segment (start 169.164 88.138) (end 169.799 88.138) (width 0.4064) (layer F.Cu) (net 3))
 (segment (start 171.069 81.518) (end 173.339 81.518) (width 0.4064) (layer F.Cu) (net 3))
 (segment (start 173.339 81.518) (end 173.609 81.788) (width 0.4064) (layer F.Cu) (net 3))
 (segment (start 171.069 81.518) (end 169.434 81.518) (width 0.4064) (layer F.Cu) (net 3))
 (segment (start 169.434 81.518) (end 168.8465 82.1055) (width 0.4064) (layer F.Cu) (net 3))
 (segment (start 168.8465 82.1055) (end 168.8465 82.5805) (width 0.4064) (layer F.Cu) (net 3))
 (segment (start 171.069 84.963) (end 171.069 81.518) (width 0.4064) (layer F.Cu) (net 3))
 (segment (start 171.069 86.868) (end 169.799 88.138) (width 0.4064) (layer F.Cu) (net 3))
 (segment (start 173.339 81.518) (end 173.609 81.788) (width 0.3048) (layer F.Cu) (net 3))
 (segment (start 171.069 84.82) (end 171.069 84.963) (width 0.4064) (layer F.Cu) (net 3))
 (segment (start 171.069 84.963) (end 171.069 86.868) (width 0.4064) (layer F.Cu) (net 3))
 (segment (start 168.8465 75.2805) (end 171.2265 75.2805) (width 0.4064) (layer F.Cu) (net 8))
 (segment (start 173.609 72.898) (end 176.149 72.898) (width 0.4064) (layer F.Cu) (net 8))
 (segment (start 171.2265 75.2805) (end 173.609 72.898) (width 0.4064) (layer F.Cu) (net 8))
 (segment (start 176.149 76.708) (end 176.149 72.898) (width 0.4064) (layer F.Cu) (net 8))
 (segment (start 167.5765 75.2805) (end 167.5765 72.5805) (width 0.4064) (layer F.Cu) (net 10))
 (segment (start 167.5765 72.5805) (end 169.799 70.358) (width 0.4064) (layer F.Cu) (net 10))
 (segment (start 155.829 74.803) (end 155.829 72.008) (width 0.4064) (layer F.Cu) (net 11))
 (segment (start 163.449 72.898) (end 160.274 72.898) (width 0.4064) (layer F.Cu) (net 11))
 (segment (start 158.369 74.803) (end 155.829 74.803) (width 0.4064) (layer F.Cu) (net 11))
 (segment (start 160.274 72.898) (end 158.369 74.803) (width 0.4064) (layer F.Cu) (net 11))
 (segment (start 166.3065 75.2805) (end 166.3065 73.2155) (width 0.4064) (layer F.Cu) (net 11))
 (segment (start 165.989 72.898) (end 163.449 72.898) (width 0.4064) (layer F.Cu) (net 11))
 (segment (start 166.3065 73.2155) (end 165.989 72.898) (width 0.4064) (layer F.Cu) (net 11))
 (segment (start 178.689 92.028) (end 178.689 91.868) (width 0.3048) (layer F.Cu) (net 9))
 (segment (start 178.689 91.868) (end 181.229 89.328) (width 0.3048) (layer F.Cu) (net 9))
 (segment (start 178.689 89.328) (end 178.689 88.138) (width 0.4064) (layer F.Cu) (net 6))
 (segment (start 178.689 88.138) (end 179.959 86.868) (width 0.4064) (layer F.Cu) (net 6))
 (segment (start 179.959 86.868) (end 177.419 86.868) (width 0.4064) (layer F.Cu) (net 6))
 (segment (start 177.419 86.868) (end 176.149 85.598) (width 0.4064) (layer F.Cu) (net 6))
 (segment (start 179.959 86.868) (end 179.959 87.122) (width 0.3048) (layer F.Cu) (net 6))
 (segment (start 176.149 85.598) (end 176.149 81.788) (width 0.4064) (layer F.Cu) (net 6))
 (segment (start 172.069 84.328) (end 174.244 84.328) (width 0.4064) (layer F.Cu) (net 6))
 (segment (start 174.244 84.328) (end 176.149 82.423) (width 0.4064) (layer F.Cu) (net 6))
 (segment (start 176.149 82.423) (end 176.149 81.788) (width 0.4064) (layer F.Cu) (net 6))
 (segment (start 166.3065 82.5805) (end 166.3065 84.0105) (width 0.4064) (layer F.Cu) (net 6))
 (segment (start 166.624 84.328) (end 170.069 84.328) (width 0.4064) (layer F.Cu) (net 6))
 (segment (start 166.3065 84.0105) (end 166.624 84.328) (width 0.4064) (layer F.Cu) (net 6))
 (segment (start 176.149 85.598) (end 175.895 85.598) (width 0.3048) (layer F.Cu) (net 6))
 (segment (start 176.149 79.248) (end 178.689 79.248) (width 0.4064) (layer F.Cu) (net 5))
 (segment (start 176.149 79.248) (end 174.879 80.518) (width 0.4064) (layer F.Cu) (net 5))
 (segment (start 167.5765 80.8355) (end 167.5765 82.5805) (width 0.4064) (layer F.Cu) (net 5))
 (segment (start 167.894 80.518) (end 167.5765 80.8355) (width 0.4064) (layer F.Cu) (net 5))
 (segment (start 174.879 80.518) (end 167.894 80.518) (width 0.4064) (layer F.Cu) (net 5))
 (segment (start 178.689 79.248) (end 180.594 77.343) (width 0.4064) (layer F.Cu) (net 5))
 (segment (start 180.594 77.343) (end 180.594 72.898) (width 0.4064) (layer F.Cu) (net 5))
 (segment (start 180.594 69.088) (end 180.594 72.898) (width 0.4064) (layer F.Cu) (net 5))
 (segment (start 180.594 72.898) (end 180.594 72.588) (width 0.3048) (layer F.Cu) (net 5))
 (segment (start 180.848 73.152) (end 180.594 72.898) (width 0.3048) (layer F.Cu) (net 5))
 (segment (start 171.704 77.343) (end 171.958 77.343) (width 0.4064) (layer F.Cu) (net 7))
 (segment (start 171.704 77.343) (end 170.18 77.343) (width 0.4064) (layer F.Cu) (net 7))
 (segment (start 170.18 77.343) (end 168.275 79.248) (width 0.4064) (layer F.Cu) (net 7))
 (segment (start 168.275 79.248) (end 166.624 79.248) (width 0.4064) (layer F.Cu) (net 7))
 (segment (start 166.624 79.248) (end 165.0365 80.8355) (width 0.4064) (layer F.Cu) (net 7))
 (segment (start 165.0365 82.5805) (end 165.0365 80.8355) (width 0.4064) (layer F.Cu) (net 7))
 (segment (start 171.958 77.343) (end 173.609 78.994) (width 0.4064) (layer F.Cu) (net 7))
 (segment (start 173.609 78.994) (end 173.609 79.248) (width 0.4064) (layer F.Cu) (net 7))
 (segment (start 154.559 81.788) (end 154.559 83.838) (width 0.4064) (layer F.Cu) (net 7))
 (segment (start 154.8765 83.5205) (end 154.8765 84.6455) (width 0.4064) (layer F.Cu) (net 7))
 (segment (start 155.829 85.598) (end 163.449 85.598) (width 0.4064) (layer F.Cu) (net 7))
 (segment (start 154.8765 84.6455) (end 155.829 85.598) (width 0.4064) (layer F.Cu) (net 7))
 (segment (start 165.0365 82.5805) (end 165.0365 84.0105) (width 0.4064) (layer F.Cu) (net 7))
 (segment (start 165.0365 84.0105) (end 163.449 85.598) (width 0.4064) (layer F.Cu) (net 7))
 (segment (start 173.609 79.248) (end 173.609 78.994) (width 0.3048) (layer F.Cu) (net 7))
 (segment (start 160.909 93.218) (end 160.909 91.948) (width 0.4064) (layer F.Cu) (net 2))
 (segment (start 150.749 88.773) (end 146.304 93.218) (width 0.4064) (layer F.Cu) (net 2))
 (segment (start 157.734 88.773) (end 150.749 88.773) (width 0.4064) (layer F.Cu) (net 2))
 (segment (start 160.909 91.948) (end 157.734 88.773) (width 0.4064) (layer F.Cu) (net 2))
 (segment (start 164.759 90.678) (end 163.449 90.678) (width 0.4064) (layer F.Cu) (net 2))
 (segment (start 163.449 90.678) (end 160.909 93.218) (width 0.4064) (layer F.Cu) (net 2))
 (segment (start 133.604 93.218) (end 139.694 93.218) (width 0.4064) (layer F.Cu) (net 2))
 (segment (start 139.694 93.218) (end 139.954 93.478) (width 0.4064) (layer F.Cu) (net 2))
 (segment (start 146.304 93.218) (end 140.214 93.218) (width 0.4064) (layer F.Cu) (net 2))
 (segment (start 140.214 93.218) (end 139.954 93.478) (width 0.4064) (layer F.Cu) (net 2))
 (segment (start 140.214 93.218) (end 139.954 93.478) (width 0.4064) (layer F.Cu) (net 2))
 (segment (start 139.694 93.218) (end 139.954 93.478) (width 0.4064) (layer F.Cu) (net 2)))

